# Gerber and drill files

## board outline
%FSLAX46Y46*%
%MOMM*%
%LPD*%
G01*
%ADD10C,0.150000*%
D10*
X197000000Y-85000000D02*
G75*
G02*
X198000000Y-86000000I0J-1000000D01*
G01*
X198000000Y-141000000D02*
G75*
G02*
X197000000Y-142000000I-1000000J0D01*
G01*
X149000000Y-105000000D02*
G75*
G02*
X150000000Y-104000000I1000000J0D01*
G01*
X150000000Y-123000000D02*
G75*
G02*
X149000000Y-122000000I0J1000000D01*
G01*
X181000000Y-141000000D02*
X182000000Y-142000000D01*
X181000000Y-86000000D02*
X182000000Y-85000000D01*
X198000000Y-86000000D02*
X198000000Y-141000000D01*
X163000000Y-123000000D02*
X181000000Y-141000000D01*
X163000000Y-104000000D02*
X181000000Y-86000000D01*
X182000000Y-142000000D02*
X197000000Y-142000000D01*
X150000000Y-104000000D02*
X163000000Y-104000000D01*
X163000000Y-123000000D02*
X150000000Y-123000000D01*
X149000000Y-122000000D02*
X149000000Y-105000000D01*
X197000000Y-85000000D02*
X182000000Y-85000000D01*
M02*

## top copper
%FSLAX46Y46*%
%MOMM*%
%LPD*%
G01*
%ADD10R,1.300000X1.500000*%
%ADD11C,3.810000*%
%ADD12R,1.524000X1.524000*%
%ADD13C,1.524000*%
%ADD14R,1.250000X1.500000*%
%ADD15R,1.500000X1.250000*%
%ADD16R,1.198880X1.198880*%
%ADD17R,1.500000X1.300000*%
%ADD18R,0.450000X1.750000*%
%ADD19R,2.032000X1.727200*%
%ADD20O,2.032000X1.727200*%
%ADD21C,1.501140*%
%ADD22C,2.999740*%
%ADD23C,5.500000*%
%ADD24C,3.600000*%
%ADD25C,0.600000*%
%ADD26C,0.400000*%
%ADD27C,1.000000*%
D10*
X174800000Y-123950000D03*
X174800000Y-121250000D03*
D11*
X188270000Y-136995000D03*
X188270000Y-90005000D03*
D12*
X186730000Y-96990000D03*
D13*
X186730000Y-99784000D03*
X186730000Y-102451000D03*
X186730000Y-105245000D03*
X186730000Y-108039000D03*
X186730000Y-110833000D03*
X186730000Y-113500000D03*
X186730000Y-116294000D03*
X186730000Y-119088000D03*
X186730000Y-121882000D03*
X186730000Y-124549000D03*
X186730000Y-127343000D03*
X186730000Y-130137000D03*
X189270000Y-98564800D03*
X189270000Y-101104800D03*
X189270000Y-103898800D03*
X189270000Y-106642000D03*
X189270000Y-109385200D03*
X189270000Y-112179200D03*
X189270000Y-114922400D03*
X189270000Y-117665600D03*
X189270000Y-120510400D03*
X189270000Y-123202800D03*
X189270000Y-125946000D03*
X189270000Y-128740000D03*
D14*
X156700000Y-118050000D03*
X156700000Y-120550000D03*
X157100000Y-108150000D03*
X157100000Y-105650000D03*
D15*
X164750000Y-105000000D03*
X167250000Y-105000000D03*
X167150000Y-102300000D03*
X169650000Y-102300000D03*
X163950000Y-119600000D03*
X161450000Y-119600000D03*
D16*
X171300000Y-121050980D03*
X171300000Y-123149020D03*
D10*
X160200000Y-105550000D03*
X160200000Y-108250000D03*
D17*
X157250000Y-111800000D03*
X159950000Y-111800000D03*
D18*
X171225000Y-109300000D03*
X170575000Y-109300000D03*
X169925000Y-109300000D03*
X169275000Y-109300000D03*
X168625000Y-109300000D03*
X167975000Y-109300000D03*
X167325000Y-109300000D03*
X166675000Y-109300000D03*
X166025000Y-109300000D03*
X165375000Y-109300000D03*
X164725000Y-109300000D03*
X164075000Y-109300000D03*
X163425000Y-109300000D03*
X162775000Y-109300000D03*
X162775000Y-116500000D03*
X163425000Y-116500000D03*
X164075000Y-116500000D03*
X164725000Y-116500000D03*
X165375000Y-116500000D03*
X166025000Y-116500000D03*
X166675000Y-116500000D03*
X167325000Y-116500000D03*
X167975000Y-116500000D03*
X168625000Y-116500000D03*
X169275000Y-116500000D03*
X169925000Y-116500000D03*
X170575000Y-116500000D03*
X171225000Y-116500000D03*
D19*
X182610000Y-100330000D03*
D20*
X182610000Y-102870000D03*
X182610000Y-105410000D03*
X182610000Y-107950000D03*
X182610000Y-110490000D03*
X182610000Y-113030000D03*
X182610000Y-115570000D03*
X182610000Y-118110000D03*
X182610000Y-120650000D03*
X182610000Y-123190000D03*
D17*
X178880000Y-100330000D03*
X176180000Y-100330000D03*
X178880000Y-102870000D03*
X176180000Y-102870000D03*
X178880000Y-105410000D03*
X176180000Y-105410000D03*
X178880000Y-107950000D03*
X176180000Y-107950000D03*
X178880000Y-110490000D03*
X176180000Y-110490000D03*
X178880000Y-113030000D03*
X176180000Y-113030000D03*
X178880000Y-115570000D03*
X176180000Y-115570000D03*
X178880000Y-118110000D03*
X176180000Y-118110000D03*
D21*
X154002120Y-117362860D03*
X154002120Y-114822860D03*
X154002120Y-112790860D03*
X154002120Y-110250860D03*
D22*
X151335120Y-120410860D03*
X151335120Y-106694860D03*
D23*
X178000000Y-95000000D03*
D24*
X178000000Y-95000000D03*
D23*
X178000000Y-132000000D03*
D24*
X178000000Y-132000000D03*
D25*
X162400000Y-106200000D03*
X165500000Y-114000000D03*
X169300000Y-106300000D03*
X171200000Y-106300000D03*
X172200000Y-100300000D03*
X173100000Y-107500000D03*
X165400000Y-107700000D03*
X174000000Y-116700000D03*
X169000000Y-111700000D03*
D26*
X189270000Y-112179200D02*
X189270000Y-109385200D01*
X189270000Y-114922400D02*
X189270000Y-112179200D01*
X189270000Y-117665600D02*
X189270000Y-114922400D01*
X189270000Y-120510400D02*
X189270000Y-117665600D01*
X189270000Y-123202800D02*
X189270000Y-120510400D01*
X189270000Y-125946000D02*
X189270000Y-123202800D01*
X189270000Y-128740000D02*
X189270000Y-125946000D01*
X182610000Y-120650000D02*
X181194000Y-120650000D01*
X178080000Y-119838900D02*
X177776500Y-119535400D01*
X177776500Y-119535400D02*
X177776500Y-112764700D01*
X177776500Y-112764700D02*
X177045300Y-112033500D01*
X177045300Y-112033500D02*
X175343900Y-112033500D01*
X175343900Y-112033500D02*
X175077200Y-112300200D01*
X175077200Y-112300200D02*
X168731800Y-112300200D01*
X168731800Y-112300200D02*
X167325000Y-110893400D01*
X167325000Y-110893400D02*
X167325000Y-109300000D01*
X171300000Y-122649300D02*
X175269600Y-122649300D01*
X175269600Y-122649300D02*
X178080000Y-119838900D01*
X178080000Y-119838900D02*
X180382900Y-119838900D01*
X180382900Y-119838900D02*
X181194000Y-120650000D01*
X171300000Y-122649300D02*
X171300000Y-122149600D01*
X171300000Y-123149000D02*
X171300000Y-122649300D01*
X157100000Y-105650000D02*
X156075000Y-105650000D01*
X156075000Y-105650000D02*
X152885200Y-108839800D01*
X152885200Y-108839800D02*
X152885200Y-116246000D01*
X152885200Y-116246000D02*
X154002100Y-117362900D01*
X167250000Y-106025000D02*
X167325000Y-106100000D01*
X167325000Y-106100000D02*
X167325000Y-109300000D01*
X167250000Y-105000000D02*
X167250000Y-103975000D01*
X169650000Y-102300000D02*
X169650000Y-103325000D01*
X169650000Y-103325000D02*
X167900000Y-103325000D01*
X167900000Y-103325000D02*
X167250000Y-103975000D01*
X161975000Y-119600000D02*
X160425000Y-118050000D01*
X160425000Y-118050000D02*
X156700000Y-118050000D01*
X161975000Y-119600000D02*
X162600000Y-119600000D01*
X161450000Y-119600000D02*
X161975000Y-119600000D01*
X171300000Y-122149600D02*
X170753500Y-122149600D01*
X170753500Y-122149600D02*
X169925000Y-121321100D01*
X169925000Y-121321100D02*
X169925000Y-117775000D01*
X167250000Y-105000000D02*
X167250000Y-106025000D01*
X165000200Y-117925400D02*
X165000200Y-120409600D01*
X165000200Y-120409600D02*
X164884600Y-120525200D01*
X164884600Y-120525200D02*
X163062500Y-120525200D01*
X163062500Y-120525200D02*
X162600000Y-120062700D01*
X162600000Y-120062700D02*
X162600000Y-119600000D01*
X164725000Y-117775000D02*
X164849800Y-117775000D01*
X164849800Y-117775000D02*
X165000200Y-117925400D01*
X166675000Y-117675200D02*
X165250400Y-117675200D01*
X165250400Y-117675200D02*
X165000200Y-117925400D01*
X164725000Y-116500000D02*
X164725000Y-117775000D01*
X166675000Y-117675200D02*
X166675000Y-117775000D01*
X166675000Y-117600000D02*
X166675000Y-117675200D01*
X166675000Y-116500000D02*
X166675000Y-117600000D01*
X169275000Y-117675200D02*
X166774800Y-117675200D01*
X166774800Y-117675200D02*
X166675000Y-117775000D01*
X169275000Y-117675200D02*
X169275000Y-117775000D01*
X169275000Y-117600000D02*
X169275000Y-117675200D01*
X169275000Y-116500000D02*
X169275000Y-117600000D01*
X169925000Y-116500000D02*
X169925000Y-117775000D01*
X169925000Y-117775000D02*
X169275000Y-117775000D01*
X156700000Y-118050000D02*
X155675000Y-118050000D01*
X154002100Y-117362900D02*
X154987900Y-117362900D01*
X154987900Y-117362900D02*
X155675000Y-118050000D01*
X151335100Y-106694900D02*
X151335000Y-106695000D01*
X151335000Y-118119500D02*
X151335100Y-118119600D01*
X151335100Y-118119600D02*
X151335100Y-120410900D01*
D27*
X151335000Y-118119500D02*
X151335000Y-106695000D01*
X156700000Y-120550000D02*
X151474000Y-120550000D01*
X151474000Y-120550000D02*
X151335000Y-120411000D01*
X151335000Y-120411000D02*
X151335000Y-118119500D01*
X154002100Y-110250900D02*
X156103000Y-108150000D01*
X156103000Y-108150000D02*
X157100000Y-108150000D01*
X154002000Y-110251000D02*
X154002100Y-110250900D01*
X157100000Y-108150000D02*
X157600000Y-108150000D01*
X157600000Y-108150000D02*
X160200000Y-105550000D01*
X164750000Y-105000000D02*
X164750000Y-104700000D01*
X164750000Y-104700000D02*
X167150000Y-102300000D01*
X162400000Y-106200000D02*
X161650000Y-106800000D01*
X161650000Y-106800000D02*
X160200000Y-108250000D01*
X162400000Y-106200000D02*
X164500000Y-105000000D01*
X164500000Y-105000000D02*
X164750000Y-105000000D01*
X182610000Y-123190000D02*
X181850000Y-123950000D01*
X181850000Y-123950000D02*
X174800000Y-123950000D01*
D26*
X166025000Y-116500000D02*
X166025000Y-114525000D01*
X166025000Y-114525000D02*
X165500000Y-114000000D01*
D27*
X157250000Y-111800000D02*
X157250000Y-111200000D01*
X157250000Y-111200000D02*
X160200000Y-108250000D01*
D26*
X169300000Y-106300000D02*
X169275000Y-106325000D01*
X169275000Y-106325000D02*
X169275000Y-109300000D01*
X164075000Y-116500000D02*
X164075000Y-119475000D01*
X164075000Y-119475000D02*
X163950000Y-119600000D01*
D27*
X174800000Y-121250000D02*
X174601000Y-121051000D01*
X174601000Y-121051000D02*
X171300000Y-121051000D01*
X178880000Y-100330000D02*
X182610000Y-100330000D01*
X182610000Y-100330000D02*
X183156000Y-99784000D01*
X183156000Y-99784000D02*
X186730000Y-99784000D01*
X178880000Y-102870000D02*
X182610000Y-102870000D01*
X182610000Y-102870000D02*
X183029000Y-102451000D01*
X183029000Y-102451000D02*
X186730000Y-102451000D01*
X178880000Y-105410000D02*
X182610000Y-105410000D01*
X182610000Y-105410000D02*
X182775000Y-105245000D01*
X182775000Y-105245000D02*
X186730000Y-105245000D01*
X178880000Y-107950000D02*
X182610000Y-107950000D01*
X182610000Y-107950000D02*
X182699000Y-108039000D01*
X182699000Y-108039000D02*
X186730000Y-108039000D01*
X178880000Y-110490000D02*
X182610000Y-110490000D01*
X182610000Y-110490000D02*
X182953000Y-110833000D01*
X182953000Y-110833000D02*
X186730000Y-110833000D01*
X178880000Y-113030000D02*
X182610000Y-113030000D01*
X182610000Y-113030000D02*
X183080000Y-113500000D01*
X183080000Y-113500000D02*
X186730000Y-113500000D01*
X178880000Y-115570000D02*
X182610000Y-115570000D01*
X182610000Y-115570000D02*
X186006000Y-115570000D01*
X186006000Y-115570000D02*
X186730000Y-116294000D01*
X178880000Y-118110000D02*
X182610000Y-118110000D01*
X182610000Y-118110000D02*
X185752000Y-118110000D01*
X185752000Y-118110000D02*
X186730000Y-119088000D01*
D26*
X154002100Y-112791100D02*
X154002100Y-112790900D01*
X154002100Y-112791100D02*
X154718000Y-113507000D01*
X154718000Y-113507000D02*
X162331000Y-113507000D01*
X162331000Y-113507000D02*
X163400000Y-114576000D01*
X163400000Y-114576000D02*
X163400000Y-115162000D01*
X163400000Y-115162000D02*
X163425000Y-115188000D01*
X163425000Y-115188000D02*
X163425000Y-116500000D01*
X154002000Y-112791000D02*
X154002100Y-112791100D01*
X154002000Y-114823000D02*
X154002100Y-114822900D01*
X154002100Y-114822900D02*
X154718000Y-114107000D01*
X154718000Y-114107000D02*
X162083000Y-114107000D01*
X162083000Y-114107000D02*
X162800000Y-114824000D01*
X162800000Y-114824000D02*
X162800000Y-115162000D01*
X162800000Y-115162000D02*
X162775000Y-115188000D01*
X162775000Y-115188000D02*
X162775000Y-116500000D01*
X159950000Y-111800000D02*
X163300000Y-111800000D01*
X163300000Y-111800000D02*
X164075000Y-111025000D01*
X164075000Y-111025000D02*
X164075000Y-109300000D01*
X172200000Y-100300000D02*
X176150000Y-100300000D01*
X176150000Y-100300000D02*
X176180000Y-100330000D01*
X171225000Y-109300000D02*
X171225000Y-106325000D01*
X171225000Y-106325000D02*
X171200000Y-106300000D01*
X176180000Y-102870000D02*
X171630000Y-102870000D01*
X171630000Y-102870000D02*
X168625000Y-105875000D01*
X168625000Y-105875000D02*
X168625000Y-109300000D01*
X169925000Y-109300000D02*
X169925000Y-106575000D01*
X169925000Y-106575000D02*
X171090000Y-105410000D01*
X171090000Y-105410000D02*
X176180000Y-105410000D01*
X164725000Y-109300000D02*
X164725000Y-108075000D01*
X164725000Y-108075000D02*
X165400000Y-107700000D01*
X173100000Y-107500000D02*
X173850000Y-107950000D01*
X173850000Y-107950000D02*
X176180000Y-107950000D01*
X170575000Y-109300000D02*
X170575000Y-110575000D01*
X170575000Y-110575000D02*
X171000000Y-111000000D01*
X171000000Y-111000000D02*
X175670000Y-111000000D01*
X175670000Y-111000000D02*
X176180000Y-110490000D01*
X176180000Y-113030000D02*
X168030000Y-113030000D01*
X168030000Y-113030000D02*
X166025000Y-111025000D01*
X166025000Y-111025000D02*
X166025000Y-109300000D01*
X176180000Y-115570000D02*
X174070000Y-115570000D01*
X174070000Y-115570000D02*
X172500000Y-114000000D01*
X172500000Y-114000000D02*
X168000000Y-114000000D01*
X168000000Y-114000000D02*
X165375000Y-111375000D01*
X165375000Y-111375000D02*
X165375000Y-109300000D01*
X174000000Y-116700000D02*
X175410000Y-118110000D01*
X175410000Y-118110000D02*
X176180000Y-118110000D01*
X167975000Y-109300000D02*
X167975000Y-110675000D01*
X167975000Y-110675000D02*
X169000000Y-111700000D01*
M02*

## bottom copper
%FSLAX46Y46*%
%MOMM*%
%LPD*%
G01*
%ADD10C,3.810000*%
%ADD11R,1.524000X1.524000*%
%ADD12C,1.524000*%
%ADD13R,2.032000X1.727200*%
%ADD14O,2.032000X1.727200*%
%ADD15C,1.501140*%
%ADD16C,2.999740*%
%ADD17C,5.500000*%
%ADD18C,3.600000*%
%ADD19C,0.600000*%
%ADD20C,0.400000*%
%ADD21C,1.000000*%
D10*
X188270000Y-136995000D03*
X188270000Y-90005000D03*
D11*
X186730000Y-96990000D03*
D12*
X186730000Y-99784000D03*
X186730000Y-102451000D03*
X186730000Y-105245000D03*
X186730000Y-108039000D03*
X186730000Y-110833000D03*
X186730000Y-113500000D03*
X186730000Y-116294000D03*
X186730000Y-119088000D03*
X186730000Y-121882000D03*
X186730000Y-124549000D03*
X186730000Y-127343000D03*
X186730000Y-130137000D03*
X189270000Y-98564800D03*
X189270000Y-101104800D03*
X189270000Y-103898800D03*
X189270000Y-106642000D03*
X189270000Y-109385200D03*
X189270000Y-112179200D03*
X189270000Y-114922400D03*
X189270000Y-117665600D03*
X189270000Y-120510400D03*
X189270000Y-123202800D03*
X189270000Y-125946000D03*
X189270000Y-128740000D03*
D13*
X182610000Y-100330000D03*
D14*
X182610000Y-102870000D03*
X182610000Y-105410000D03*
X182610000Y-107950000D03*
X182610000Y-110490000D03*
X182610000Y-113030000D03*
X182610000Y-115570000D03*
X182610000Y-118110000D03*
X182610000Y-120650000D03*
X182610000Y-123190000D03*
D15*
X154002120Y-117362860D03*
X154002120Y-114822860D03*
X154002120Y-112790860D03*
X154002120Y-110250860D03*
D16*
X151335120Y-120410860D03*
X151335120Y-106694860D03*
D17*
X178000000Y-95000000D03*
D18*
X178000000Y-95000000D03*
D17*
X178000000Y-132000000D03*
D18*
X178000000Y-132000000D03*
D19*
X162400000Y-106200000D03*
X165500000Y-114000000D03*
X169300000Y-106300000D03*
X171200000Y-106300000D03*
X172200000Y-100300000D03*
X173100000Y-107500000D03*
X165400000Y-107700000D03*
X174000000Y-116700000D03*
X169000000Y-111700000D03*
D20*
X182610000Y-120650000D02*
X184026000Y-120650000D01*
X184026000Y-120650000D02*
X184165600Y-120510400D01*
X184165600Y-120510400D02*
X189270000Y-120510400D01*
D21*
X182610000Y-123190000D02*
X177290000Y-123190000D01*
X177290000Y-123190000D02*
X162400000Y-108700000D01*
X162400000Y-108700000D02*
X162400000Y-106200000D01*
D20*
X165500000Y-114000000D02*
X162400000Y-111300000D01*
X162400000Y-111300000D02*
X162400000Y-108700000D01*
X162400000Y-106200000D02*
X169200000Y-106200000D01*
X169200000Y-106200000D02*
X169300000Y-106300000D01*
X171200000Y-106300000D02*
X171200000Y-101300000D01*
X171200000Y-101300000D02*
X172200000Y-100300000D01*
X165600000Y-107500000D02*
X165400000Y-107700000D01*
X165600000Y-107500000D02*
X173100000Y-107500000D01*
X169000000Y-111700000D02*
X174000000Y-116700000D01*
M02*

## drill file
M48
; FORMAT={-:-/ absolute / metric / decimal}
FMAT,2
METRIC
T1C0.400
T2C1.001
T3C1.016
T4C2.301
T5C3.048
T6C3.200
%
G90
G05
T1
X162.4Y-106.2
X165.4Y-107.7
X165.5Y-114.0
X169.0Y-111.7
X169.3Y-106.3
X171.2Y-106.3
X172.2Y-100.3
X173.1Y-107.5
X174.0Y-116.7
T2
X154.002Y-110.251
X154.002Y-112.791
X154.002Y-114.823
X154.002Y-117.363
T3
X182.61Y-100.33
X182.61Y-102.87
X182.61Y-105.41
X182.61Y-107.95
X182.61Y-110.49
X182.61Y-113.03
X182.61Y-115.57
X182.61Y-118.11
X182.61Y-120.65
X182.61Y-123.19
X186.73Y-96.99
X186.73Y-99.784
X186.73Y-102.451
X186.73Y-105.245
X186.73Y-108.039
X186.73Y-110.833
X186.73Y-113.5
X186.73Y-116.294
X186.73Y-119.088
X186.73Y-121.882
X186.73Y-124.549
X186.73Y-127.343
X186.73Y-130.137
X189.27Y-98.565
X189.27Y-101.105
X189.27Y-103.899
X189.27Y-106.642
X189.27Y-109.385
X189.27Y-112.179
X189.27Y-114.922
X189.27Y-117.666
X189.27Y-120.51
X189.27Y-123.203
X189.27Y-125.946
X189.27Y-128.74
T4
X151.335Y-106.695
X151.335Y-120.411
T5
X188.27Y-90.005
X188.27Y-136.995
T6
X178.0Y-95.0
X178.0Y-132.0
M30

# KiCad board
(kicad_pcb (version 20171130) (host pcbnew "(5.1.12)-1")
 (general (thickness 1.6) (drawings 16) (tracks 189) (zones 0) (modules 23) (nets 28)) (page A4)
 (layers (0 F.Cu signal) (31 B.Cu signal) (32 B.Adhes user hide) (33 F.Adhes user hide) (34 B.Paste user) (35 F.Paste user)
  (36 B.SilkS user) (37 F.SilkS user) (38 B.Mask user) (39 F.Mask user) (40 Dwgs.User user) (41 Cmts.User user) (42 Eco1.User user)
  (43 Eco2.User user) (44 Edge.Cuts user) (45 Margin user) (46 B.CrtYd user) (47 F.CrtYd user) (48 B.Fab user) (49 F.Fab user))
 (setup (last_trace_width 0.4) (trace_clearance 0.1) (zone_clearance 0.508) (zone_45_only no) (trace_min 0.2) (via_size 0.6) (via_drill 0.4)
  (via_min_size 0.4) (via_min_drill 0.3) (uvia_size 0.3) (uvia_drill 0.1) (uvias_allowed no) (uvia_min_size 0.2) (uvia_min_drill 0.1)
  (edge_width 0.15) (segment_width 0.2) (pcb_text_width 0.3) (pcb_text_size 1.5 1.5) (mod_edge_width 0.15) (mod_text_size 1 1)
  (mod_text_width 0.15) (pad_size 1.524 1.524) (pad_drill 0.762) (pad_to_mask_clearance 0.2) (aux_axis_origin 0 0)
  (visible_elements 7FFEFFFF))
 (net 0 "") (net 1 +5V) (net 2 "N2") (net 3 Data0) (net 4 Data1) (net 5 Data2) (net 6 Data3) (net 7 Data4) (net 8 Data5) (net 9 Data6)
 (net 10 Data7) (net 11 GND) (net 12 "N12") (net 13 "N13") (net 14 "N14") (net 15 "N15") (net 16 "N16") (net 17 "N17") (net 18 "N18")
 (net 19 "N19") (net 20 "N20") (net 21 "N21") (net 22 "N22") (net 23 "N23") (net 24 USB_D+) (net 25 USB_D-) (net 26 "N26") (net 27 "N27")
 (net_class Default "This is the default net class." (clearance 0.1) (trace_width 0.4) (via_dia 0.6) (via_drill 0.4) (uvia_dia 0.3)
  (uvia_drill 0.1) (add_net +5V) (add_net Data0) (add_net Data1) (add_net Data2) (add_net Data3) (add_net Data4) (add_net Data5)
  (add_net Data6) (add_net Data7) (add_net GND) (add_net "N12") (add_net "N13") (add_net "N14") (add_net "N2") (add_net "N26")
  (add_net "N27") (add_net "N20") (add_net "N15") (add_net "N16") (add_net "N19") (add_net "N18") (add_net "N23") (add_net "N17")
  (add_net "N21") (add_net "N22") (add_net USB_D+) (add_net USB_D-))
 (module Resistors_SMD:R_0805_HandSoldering (layer F.Cu) (at 174.8 122.6 90)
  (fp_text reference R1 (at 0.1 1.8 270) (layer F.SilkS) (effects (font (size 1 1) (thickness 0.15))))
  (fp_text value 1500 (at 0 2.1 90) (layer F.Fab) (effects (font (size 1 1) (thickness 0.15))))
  (pad 1 smd rect (at -1.35 0 90) (size 1.5 1.3) (layers F.Cu F.Paste F.Mask) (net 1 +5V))
  (pad 2 smd rect (at 1.35 0 90) (size 1.5 1.3) (layers F.Cu F.Paste F.Mask) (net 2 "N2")))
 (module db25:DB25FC (layer F.Cu) (at 187 113.5 270)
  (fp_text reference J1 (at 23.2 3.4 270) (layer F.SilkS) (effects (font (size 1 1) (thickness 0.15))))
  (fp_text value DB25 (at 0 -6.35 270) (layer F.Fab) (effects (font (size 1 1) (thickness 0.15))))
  (pad "" thru_hole circle (at 23.495 -1.27 270) (size 3.81 3.81) (drill 3.048) (layers *.Cu *.Mask F.SilkS))
  (pad "" thru_hole circle (at -23.495 -1.27 270) (size 3.81 3.81) (drill 3.048) (layers *.Cu *.Mask F.SilkS))
  (pad 1 thru_hole rect (at -16.51 0.27 270) (size 1.524 1.524) (drill 1.016) (layers *.Cu *.Mask F.SilkS))
  (pad 2 thru_hole circle (at -13.716 0.27 270) (size 1.524 1.524) (drill 1.016) (layers *.Cu *.Mask F.SilkS) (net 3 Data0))
  (pad 3 thru_hole circle (at -11.049 0.27 270) (size 1.524 1.524) (drill 1.016) (layers *.Cu *.Mask F.SilkS) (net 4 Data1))
  (pad 4 thru_hole circle (at -8.255 0.27 270) (size 1.524 1.524) (drill 1.016) (layers *.Cu *.Mask F.SilkS) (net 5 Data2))
  (pad 5 thru_hole circle (at -5.461 0.27 270) (size 1.524 1.524) (drill 1.016) (layers *.Cu *.Mask F.SilkS) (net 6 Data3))
  (pad 6 thru_hole circle (at -2.667 0.27 270) (size 1.524 1.524) (drill 1.016) (layers *.Cu *.Mask F.SilkS) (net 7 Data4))
  (pad 7 thru_hole circle (at 0 0.27 270) (size 1.524 1.524) (drill 1.016) (layers *.Cu *.Mask F.SilkS) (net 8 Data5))
  (pad 8 thru_hole circle (at 2.794 0.27 270) (size 1.524 1.524) (drill 1.016) (layers *.Cu *.Mask F.SilkS) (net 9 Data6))
  (pad 9 thru_hole circle (at 5.588 0.27 270) (size 1.524 1.524) (drill 1.016) (layers *.Cu *.Mask F.SilkS) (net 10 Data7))
  (pad 10 thru_hole circle (at 8.382 0.27 270) (size 1.524 1.524) (drill 1.016) (layers *.Cu *.Mask F.SilkS))
  (pad 11 thru_hole circle (at 11.049 0.27 270) (size 1.524 1.524) (drill 1.016) (layers *.Cu *.Mask F.SilkS))
  (pad 12 thru_hole circle (at 13.843 0.27 270) (size 1.524 1.524) (drill 1.016) (layers *.Cu *.Mask F.SilkS))
  (pad 13 thru_hole circle (at 16.637 0.27 270) (size 1.524 1.524) (drill 1.016) (layers *.Cu *.Mask F.SilkS))
  (pad 14 thru_hole circle (at -14.9352 -2.27 270) (size 1.524 1.524) (drill 1.016) (layers *.Cu *.Mask F.SilkS))
  (pad 15 thru_hole circle (at -12.3952 -2.27 270) (size 1.524 1.524) (drill 1.016) (layers *.Cu *.Mask F.SilkS))
  (pad 16 thru_hole circle (at -9.6012 -2.27 270) (size 1.524 1.524) (drill 1.016) (layers *.Cu *.Mask F.SilkS))
  (pad 17 thru_hole circle (at -6.858 -2.27 270) (size 1.524 1.524) (drill 1.016) (layers *.Cu *.Mask F.SilkS))
  (pad 18 thru_hole circle (at -4.1148 -2.27 270) (size 1.524 1.524) (drill 1.016) (layers *.Cu *.Mask F.SilkS) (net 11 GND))
  (pad 19 thru_hole circle (at -1.3208 -2.27 270) (size 1.524 1.524) (drill 1.016) (layers *.Cu *.Mask F.SilkS) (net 11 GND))
  (pad 20 thru_hole circle (at 1.4224 -2.27 270) (size 1.524 1.524) (drill 1.016) (layers *.Cu *.Mask F.SilkS) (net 11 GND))
  (pad 21 thru_hole circle (at 4.1656 -2.27 270) (size 1.524 1.524) (drill 1.016) (layers *.Cu *.Mask F.SilkS) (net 11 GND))
  (pad 22 thru_hole circle (at 7.0104 -2.27 270) (size 1.524 1.524) (drill 1.016) (layers *.Cu *.Mask F.SilkS) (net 11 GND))
  (pad 23 thru_hole circle (at 9.7028 -2.27 270) (size 1.524 1.524) (drill 1.016) (layers *.Cu *.Mask F.SilkS) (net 11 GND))
  (pad 24 thru_hole circle (at 12.446 -2.27 270) (size 1.524 1.524) (drill 1.016) (layers *.Cu *.Mask F.SilkS) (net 11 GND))
  (pad 25 thru_hole circle (at 15.24 -2.27 270) (size 1.524 1.524) (drill 1.016) (layers *.Cu *.Mask F.SilkS) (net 11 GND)))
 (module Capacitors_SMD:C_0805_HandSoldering (layer F.Cu) (at 156.7 119.3 270)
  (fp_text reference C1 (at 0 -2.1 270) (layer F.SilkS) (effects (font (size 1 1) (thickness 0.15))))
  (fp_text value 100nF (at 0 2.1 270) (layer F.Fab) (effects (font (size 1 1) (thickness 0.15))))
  (pad 1 smd rect (at -1.25 0 270) (size 1.5 1.25) (layers F.Cu F.Paste F.Mask) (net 11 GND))
  (pad 2 smd rect (at 1.25 0 270) (size 1.5 1.25) (layers F.Cu F.Paste F.Mask) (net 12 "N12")))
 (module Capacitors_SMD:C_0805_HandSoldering (layer F.Cu) (at 157.1 106.9 90)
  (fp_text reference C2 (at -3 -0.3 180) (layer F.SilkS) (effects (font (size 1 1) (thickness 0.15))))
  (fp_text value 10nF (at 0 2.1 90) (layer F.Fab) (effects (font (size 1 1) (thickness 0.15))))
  (pad 1 smd rect (at -1.25 0 90) (size 1.5 1.25) (layers F.Cu F.Paste F.Mask) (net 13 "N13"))
  (pad 2 smd rect (at 1.25 0 90) (size 1.5 1.25) (layers F.Cu F.Paste F.Mask) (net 11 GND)))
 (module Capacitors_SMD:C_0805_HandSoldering (layer F.Cu) (at 166 105)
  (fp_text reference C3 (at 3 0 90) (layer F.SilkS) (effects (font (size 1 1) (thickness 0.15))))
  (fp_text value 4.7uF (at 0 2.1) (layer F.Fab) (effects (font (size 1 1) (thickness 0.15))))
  (pad 1 smd rect (at -1.25 0) (size 1.5 1.25) (layers F.Cu F.Paste F.Mask) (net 1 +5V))
  (pad 2 smd rect (at 1.25 0) (size 1.5 1.25) (layers F.Cu F.Paste F.Mask) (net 11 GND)))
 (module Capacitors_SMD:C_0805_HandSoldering (layer F.Cu) (at 168.4 102.3)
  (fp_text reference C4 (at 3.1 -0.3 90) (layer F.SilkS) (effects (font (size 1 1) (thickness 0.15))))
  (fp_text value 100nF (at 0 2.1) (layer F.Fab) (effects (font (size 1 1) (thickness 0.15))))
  (pad 1 smd rect (at -1.25 0) (size 1.5 1.25) (layers F.Cu F.Paste F.Mask) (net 1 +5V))
  (pad 2 smd rect (at 1.25 0) (size 1.5 1.25) (layers F.Cu F.Paste F.Mask) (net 11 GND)))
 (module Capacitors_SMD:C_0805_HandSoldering (layer F.Cu) (at 162.7 119.6 180)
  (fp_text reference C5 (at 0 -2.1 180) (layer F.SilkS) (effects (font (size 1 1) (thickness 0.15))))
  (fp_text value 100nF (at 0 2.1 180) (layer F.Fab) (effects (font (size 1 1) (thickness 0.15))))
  (pad 1 smd rect (at -1.25 0 180) (size 1.5 1.25) (layers F.Cu F.Paste F.Mask) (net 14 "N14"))
  (pad 2 smd rect (at 1.25 0 180) (size 1.5 1.25) (layers F.Cu F.Paste F.Mask) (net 11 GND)))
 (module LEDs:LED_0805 (layer F.Cu) (at 171.3 122.1 90)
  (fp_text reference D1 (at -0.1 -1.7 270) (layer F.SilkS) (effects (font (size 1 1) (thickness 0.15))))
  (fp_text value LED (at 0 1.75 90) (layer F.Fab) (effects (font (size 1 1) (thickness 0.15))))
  (pad 2 smd rect (at 1.04902 0 270) (size 1.19888 1.19888) (layers F.Cu F.Paste F.Mask) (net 2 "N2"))
  (pad 1 smd rect (at -1.04902 0 270) (size 1.19888 1.19888) (layers F.Cu F.Paste F.Mask) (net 11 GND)))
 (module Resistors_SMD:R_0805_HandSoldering (layer F.Cu) (at 160.2 106.9 270)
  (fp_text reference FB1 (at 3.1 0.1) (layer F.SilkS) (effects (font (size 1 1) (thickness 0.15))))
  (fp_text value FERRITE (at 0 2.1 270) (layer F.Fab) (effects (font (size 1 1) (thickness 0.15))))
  (pad 1 smd rect (at -1.35 0 270) (size 1.5 1.3) (layers F.Cu F.Paste F.Mask) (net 13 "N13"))
  (pad 2 smd rect (at 1.35 0 270) (size 1.5 1.3) (layers F.Cu F.Paste F.Mask) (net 1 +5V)))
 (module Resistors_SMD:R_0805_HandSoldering (layer F.Cu) (at 158.6 111.8)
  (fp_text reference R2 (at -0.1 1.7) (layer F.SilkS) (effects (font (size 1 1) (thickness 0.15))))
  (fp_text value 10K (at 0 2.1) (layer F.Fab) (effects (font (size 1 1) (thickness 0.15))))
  (pad 1 smd rect (at -1.35 0) (size 1.5 1.3) (layers F.Cu F.Paste F.Mask) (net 1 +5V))
  (pad 2 smd rect (at 1.35 0) (size 1.5 1.3) (layers F.Cu F.Paste F.Mask) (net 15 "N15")))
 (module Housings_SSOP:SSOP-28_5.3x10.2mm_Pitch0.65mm (layer F.Cu) (at 167 112.9 270)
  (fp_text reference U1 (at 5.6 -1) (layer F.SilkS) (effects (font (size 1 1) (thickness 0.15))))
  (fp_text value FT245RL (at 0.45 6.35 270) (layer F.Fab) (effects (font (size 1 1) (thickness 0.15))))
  (pad 1 smd rect (at -3.6 -4.225 270) (size 1.75 0.45) (layers F.Cu F.Paste F.Mask) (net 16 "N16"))
  (pad 2 smd rect (at -3.6 -3.575 270) (size 1.75 0.45) (layers F.Cu F.Paste F.Mask) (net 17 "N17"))
  (pad 3 smd rect (at -3.6 -2.925 270) (size 1.75 0.45) (layers F.Cu F.Paste F.Mask) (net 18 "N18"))
  (pad 4 smd rect (at -3.6 -2.275 270) (size 1.75 0.45) (layers F.Cu F.Paste F.Mask) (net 1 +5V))
  (pad 5 smd rect (at -3.6 -1.625 270) (size 1.75 0.45) (layers F.Cu F.Paste F.Mask) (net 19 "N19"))
  (pad 6 smd rect (at -3.6 -0.975 270) (size 1.75 0.45) (layers F.Cu F.Paste F.Mask) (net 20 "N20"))
  (pad 7 smd rect (at -3.6 -0.325 270) (size 1.75 0.45) (layers F.Cu F.Paste F.Mask) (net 11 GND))
  (pad 8 smd rect (at -3.6 0.325 270) (size 1.75 0.45) (layers F.Cu F.Paste F.Mask))
  (pad 9 smd rect (at -3.6 0.975 270) (size 1.75 0.45) (layers F.Cu F.Paste F.Mask) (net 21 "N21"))
  (pad 10 smd rect (at -3.6 1.625 270) (size 1.75 0.45) (layers F.Cu F.Paste F.Mask) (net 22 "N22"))
  (pad 11 smd rect (at -3.6 2.275 270) (size 1.75 0.45) (layers F.Cu F.Paste F.Mask) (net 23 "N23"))
  (pad 12 smd rect (at -3.6 2.925 270) (size 1.75 0.45) (layers F.Cu F.Paste F.Mask) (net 15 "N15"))
  (pad 13 smd rect (at -3.6 3.575 270) (size 1.75 0.45) (layers F.Cu F.Paste F.Mask))
  (pad 14 smd rect (at -3.6 4.225 270) (size 1.75 0.45) (layers F.Cu F.Paste F.Mask))
  (pad 15 smd rect (at 3.6 4.225 270) (size 1.75 0.45) (layers F.Cu F.Paste F.Mask) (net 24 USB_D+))
  (pad 16 smd rect (at 3.6 3.575 270) (size 1.75 0.45) (layers F.Cu F.Paste F.Mask) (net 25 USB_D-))
  (pad 17 smd rect (at 3.6 2.925 270) (size 1.75 0.45) (layers F.Cu F.Paste F.Mask) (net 14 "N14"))
  (pad 18 smd rect (at 3.6 2.275 270) (size 1.75 0.45) (layers F.Cu F.Paste F.Mask) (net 11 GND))
  (pad 19 smd rect (at 3.6 1.625 270) (size 1.75 0.45) (layers F.Cu F.Paste F.Mask))
  (pad 20 smd rect (at 3.6 0.975 270) (size 1.75 0.45) (layers F.Cu F.Paste F.Mask) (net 1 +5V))
  (pad 21 smd rect (at 3.6 0.325 270) (size 1.75 0.45) (layers F.Cu F.Paste F.Mask) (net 11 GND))
  (pad 22 smd rect (at 3.6 -0.325 270) (size 1.75 0.45) (layers F.Cu F.Paste F.Mask))
  (pad 23 smd rect (at 3.6 -0.975 270) (size 1.75 0.45) (layers F.Cu F.Paste F.Mask))
  (pad 24 smd rect (at 3.6 -1.625 270) (size 1.75 0.45) (layers F.Cu F.Paste F.Mask))
  (pad 25 smd rect (at 3.6 -2.275 270) (size 1.75 0.45) (layers F.Cu F.Paste F.Mask) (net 11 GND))
  (pad 26 smd rect (at 3.6 -2.925 270) (size 1.75 0.45) (layers F.Cu F.Paste F.Mask) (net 11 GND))
  (pad 27 smd rect (at 3.6 -3.575 270) (size 1.75 0.45) (layers F.Cu F.Paste F.Mask))
  (pad 28 smd rect (at 3.6 -4.225 270) (size 1.75 0.45) (layers F.Cu F.Paste F.Mask)))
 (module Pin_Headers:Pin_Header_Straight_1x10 (layer F.Cu) (at 182.61 100.33)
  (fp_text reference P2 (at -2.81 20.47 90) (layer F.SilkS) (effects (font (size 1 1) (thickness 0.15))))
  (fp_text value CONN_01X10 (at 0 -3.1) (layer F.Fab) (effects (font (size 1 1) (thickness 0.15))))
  (pad 1 thru_hole rect (at 0 0) (size 2.032 1.7272) (drill 1.016) (layers *.Cu *.Mask F.SilkS) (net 3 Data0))
  (pad 2 thru_hole oval (at 0 2.54) (size 2.032 1.7272) (drill 1.016) (layers *.Cu *.Mask F.SilkS) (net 4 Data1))
  (pad 3 thru_hole oval (at 0 5.08) (size 2.032 1.7272) (drill 1.016) (layers *.Cu *.Mask F.SilkS) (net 5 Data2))
  (pad 4 thru_hole oval (at 0 7.62) (size 2.032 1.7272) (drill 1.016) (layers *.Cu *.Mask F.SilkS) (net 6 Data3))
  (pad 5 thru_hole oval (at 0 10.16) (size 2.032 1.7272) (drill 1.016) (layers *.Cu *.Mask F.SilkS) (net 7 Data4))
  (pad 6 thru_hole oval (at 0 12.7) (size 2.032 1.7272) (drill 1.016) (layers *.Cu *.Mask F.SilkS) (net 8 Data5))
  (pad 7 thru_hole oval (at 0 15.24) (size 2.032 1.7272) (drill 1.016) (layers *.Cu *.Mask F.SilkS) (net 9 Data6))
  (pad 8 thru_hole oval (at 0 17.78) (size 2.032 1.7272) (drill 1.016) (layers *.Cu *.Mask F.SilkS) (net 10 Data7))
  (pad 9 thru_hole oval (at 0 20.32) (size 2.032 1.7272) (drill 1.016) (layers *.Cu *.Mask F.SilkS) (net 11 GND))
  (pad 10 thru_hole oval (at 0 22.86) (size 2.032 1.7272) (drill 1.016) (layers *.Cu *.Mask F.SilkS) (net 1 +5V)))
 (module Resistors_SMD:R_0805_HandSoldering (layer F.Cu) (at 177.53 100.33 180)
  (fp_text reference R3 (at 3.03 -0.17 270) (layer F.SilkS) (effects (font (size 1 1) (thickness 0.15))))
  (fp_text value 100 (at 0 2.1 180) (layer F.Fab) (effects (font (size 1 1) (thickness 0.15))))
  (pad 1 smd rect (at -1.35 0 180) (size 1.5 1.3) (layers F.Cu F.Paste F.Mask) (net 3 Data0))
  (pad 2 smd rect (at 1.35 0 180) (size 1.5 1.3) (layers F.Cu F.Paste F.Mask) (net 16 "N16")))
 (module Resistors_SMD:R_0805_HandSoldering (layer F.Cu) (at 177.53 102.87 180)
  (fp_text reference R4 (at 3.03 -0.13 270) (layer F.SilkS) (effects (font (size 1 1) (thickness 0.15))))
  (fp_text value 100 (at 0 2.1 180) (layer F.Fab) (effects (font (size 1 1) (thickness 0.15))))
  (pad 1 smd rect (at -1.35 0 180) (size 1.5 1.3) (layers F.Cu F.Paste F.Mask) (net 4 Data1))
  (pad 2 smd rect (at 1.35 0 180) (size 1.5 1.3) (layers F.Cu F.Paste F.Mask) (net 19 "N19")))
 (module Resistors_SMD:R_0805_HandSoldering (layer F.Cu) (at 177.53 105.41 180)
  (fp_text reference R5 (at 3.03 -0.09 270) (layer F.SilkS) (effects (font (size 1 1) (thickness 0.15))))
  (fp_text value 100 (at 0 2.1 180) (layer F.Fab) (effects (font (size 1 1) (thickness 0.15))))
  (pad 1 smd rect (at -1.35 0 180) (size 1.5 1.3) (layers F.Cu F.Paste F.Mask) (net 5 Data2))
  (pad 2 smd rect (at 1.35 0 180) (size 1.5 1.3) (layers F.Cu F.Paste F.Mask) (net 18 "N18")))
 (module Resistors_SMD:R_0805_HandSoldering (layer F.Cu) (at 177.53 107.95 180)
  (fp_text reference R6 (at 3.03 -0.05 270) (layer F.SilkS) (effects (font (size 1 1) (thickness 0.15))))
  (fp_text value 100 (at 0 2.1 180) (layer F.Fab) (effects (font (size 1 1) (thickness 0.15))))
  (pad 1 smd rect (at -1.35 0 180) (size 1.5 1.3) (layers F.Cu F.Paste F.Mask) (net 6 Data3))
  (pad 2 smd rect (at 1.35 0 180) (size 1.5 1.3) (layers F.Cu F.Paste F.Mask) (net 23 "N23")))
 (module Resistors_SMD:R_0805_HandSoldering (layer F.Cu) (at 177.53 110.49 180)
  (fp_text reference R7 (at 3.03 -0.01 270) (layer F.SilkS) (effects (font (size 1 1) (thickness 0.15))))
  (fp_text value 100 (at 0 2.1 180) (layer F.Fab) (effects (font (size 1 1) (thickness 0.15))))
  (pad 1 smd rect (at -1.35 0 180) (size 1.5 1.3) (layers F.Cu F.Paste F.Mask) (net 7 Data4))
  (pad 2 smd rect (at 1.35 0 180) (size 1.5 1.3) (layers F.Cu F.Paste F.Mask) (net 17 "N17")))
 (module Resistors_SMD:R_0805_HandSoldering (layer F.Cu) (at 177.53 113.03 180)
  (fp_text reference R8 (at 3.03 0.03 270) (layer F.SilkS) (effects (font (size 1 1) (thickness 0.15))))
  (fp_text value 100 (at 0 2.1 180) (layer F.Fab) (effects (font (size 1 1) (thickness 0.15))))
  (pad 1 smd rect (at -1.35 0 180) (size 1.5 1.3) (layers F.Cu F.Paste F.Mask) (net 8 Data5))
  (pad 2 smd rect (at 1.35 0 180) (size 1.5 1.3) (layers F.Cu F.Paste F.Mask) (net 21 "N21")))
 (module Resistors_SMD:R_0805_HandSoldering (layer F.Cu) (at 177.53 115.57 180)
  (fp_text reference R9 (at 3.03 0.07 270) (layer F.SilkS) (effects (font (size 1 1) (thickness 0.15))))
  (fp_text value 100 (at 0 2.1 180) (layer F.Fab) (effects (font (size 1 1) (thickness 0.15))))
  (pad 1 smd rect (at -1.35 0 180) (size 1.5 1.3) (layers F.Cu F.Paste F.Mask) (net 9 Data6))
  (pad 2 smd rect (at 1.35 0 180) (size 1.5 1.3) (layers F.Cu F.Paste F.Mask) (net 22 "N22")))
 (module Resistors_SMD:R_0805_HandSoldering (layer F.Cu) (at 177.53 118.11 180)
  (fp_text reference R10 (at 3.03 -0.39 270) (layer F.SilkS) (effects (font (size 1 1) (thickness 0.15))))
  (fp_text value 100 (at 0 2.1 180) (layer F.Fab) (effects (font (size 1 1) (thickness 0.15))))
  (pad 1 smd rect (at -1.35 0 180) (size 1.5 1.3) (layers F.Cu F.Paste F.Mask) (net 10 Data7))
  (pad 2 smd rect (at 1.35 0 180) (size 1.5 1.3) (layers F.Cu F.Paste F.Mask) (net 20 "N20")))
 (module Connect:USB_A (layer F.Cu) (at 154 110.25 270)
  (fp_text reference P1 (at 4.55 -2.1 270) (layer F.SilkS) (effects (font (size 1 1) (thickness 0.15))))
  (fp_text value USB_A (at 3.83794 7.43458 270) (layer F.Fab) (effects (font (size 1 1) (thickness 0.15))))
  (pad 4 thru_hole circle (at 7.11286 -0.00212 180) (size 1.50114 1.50114) (drill 1.00076) (layers *.Cu *.Mask F.SilkS) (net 11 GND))
  (pad 3 thru_hole circle (at 4.57286 -0.00212 180) (size 1.50114 1.50114) (drill 1.00076) (layers *.Cu *.Mask F.SilkS) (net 24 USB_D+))
  (pad 2 thru_hole circle (at 2.54086 -0.00212 180) (size 1.50114 1.50114) (drill 1.00076) (layers *.Cu *.Mask F.SilkS) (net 25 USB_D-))
  (pad 1 thru_hole circle (at 0.00086 -0.00212 180) (size 1.50114 1.50114) (drill 1.00076) (layers *.Cu *.Mask F.SilkS) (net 13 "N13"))
  (pad 5 thru_hole circle (at 10.16086 2.66488 180) (size 2.99974 2.99974) (drill 2.30124) (layers *.Cu *.Mask F.SilkS) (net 12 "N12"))
  (pad 5 thru_hole circle (at -3.55514 2.66488 180) (size 2.99974 2.99974) (drill 2.30124) (layers *.Cu *.Mask F.SilkS) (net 12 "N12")))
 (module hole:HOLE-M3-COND (layer F.Cu) (at 178 95)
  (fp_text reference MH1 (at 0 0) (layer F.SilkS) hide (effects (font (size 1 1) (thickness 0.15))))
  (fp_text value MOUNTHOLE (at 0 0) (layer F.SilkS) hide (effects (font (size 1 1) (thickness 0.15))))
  (pad 1 smd circle (at 0 0) (size 5.5 5.5) (layers F.Cu F.Mask) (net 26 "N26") (clearance 0.3) (zone_connect 2))
  (pad 1 smd circle (at 0 0) (size 5.5 5.5) (layers B.Cu B.Mask) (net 26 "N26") (clearance 0.3) (zone_connect 2))
  (pad 1 thru_hole circle (at 0 0) (size 3.6 3.6) (drill 3.2) (layers *.Cu) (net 26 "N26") (clearance 0.2) (zone_connect 2)))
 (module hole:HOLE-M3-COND (layer F.Cu) (at 178 132)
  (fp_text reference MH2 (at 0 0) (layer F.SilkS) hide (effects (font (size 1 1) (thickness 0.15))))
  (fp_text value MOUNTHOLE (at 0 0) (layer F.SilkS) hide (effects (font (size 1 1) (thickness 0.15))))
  (pad 1 smd circle (at 0 0) (size 5.5 5.5) (layers F.Cu F.Mask) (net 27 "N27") (clearance 0.3) (zone_connect 2))
  (pad 1 smd circle (at 0 0) (size 5.5 5.5) (layers B.Cu B.Mask) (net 27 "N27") (clearance 0.3) (zone_connect 2))
  (pad 1 thru_hole circle (at 0 0) (size 3.6 3.6) (drill 3.2) (layers *.Cu) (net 27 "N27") (clearance 0.2) (zone_connect 2)))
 (gr_arc (start 197 86) (end 197 85) (angle 90) (layer Edge.Cuts) (width 0.15))
 (gr_arc (start 197 141) (end 198 141) (angle 90) (layer Edge.Cuts) (width 0.15))
 (gr_arc (start 150 105) (end 149 105) (angle 90) (layer Edge.Cuts) (width 0.15))
 (gr_arc (start 150 122) (end 150 123) (angle 90) (layer Edge.Cuts) (width 0.15))
 (gr_line (start 181 141) (end 182 142) (angle 90) (layer Edge.Cuts) (width 0.15))
 (gr_line (start 181 86) (end 182 85) (angle 90) (layer Edge.Cuts) (width 0.15))
 (gr_line (start 198 86) (end 198 141) (angle 90) (layer Edge.Cuts) (width 0.15))
 (gr_line (start 163 123) (end 181 141) (angle 90) (layer Edge.Cuts) (width 0.15))
 (gr_line (start 163 104) (end 181 86) (angle 90) (layer Edge.Cuts) (width 0.15))
 (gr_line (start 182 142) (end 197 142) (angle 90) (layer Edge.Cuts) (width 0.15))
 (gr_line (start 150 104) (end 163 104) (angle 90) (layer Edge.Cuts) (width 0.15))
 (gr_line (start 163 123) (end 150 123) (angle 90) (layer Edge.Cuts) (width 0.15))
 (gr_line (start 149 122) (end 149 105) (angle 90) (layer Edge.Cuts) (width 0.15))
 (gr_line (start 197 85) (end 182 85) (angle 90) (layer Edge.Cuts) (width 0.15))
 (segment (start 189.27 112.1792) (end 189.27 109.3852) (width 0.4) (layer F.Cu) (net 11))
 (segment (start 189.27 114.9224) (end 189.27 112.1792) (width 0.4) (layer F.Cu) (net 11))
 (segment (start 189.27 117.6656) (end 189.27 114.9224) (width 0.4) (layer F.Cu) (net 11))
 (segment (start 189.27 120.5104) (end 189.27 117.6656) (width 0.4) (layer F.Cu) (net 11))
 (segment (start 189.27 123.2028) (end 189.27 120.5104) (width 0.4) (layer F.Cu) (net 11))
 (segment (start 189.27 125.946) (end 189.27 123.2028) (width 0.4) (layer F.Cu) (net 11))
 (segment (start 189.27 128.74) (end 189.27 125.946) (width 0.4) (layer F.Cu) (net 11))
 (segment (start 182.61 120.65) (end 181.194 120.65) (width 0.4) (layer F.Cu) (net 11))
 (segment (start 178.08 119.8389) (end 177.7765 119.5354) (width 0.4) (layer F.Cu) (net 11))
 (segment (start 177.7765 119.5354) (end 177.7765 112.7647) (width 0.4) (layer F.Cu) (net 11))
 (segment (start 177.7765 112.7647) (end 177.0453 112.0335) (width 0.4) (layer F.Cu) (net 11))
 (segment (start 177.0453 112.0335) (end 175.3439 112.0335) (width 0.4) (layer F.Cu) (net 11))
 (segment (start 175.3439 112.0335) (end 175.0772 112.3002) (width 0.4) (layer F.Cu) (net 11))
 (segment (start 175.0772 112.3002) (end 168.7318 112.3002) (width 0.4) (layer F.Cu) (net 11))
 (segment (start 168.7318 112.3002) (end 167.325 110.8934) (width 0.4) (layer F.Cu) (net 11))
 (segment (start 167.325 110.8934) (end 167.325 109.3) (width 0.4) (layer F.Cu) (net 11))
 (segment (start 171.3 122.6493) (end 175.2696 122.6493) (width 0.4) (layer F.Cu) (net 11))
 (segment (start 175.2696 122.6493) (end 178.08 119.8389) (width 0.4) (layer F.Cu) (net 11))
 (segment (start 178.08 119.8389) (end 180.3829 119.8389) (width 0.4) (layer F.Cu) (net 11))
 (segment (start 180.3829 119.8389) (end 181.194 120.65) (width 0.4) (layer F.Cu) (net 11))
 (segment (start 171.3 122.6493) (end 171.3 122.1496) (width 0.4) (layer F.Cu) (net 11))
 (segment (start 171.3 123.149) (end 171.3 122.6493) (width 0.4) (layer F.Cu) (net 11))
 (segment (start 157.1 105.65) (end 156.075 105.65) (width 0.4) (layer F.Cu) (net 11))
 (segment (start 156.075 105.65) (end 152.8852 108.8398) (width 0.4) (layer F.Cu) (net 11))
 (segment (start 152.8852 108.8398) (end 152.8852 116.246) (width 0.4) (layer F.Cu) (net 11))
 (segment (start 152.8852 116.246) (end 154.0021 117.3629) (width 0.4) (layer F.Cu) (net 11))
 (segment (start 167.25 106.025) (end 167.325 106.1) (width 0.4) (layer F.Cu) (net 11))
 (segment (start 167.325 106.1) (end 167.325 109.3) (width 0.4) (layer F.Cu) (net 11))
 (segment (start 167.25 105) (end 167.25 103.975) (width 0.4) (layer F.Cu) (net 11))
 (segment (start 169.65 102.3) (end 169.65 103.325) (width 0.4) (layer F.Cu) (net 11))
 (segment (start 169.65 103.325) (end 167.9 103.325) (width 0.4) (layer F.Cu) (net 11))
 (segment (start 167.9 103.325) (end 167.25 103.975) (width 0.4) (layer F.Cu) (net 11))
 (segment (start 161.975 119.6) (end 160.425 118.05) (width 0.4) (layer F.Cu) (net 11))
 (segment (start 160.425 118.05) (end 156.7 118.05) (width 0.4) (layer F.Cu) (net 11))
 (segment (start 161.975 119.6) (end 162.6 119.6) (width 0.4) (layer F.Cu) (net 11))
 (segment (start 161.45 119.6) (end 161.975 119.6) (width 0.4) (layer F.Cu) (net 11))
 (segment (start 171.3 122.1496) (end 170.7535 122.1496) (width 0.4) (layer F.Cu) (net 11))
 (segment (start 170.7535 122.1496) (end 169.925 121.3211) (width 0.4) (layer F.Cu) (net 11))
 (segment (start 169.925 121.3211) (end 169.925 117.775) (width 0.4) (layer F.Cu) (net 11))
 (segment (start 167.25 105) (end 167.25 106.025) (width 0.4) (layer F.Cu) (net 11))
 (segment (start 165.0002 117.9254) (end 165.0002 120.4096) (width 0.4) (layer F.Cu) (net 11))
 (segment (start 165.0002 120.4096) (end 164.8846 120.5252) (width 0.4) (layer F.Cu) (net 11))
 (segment (start 164.8846 120.5252) (end 163.0625 120.5252) (width 0.4) (layer F.Cu) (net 11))
 (segment (start 163.0625 120.5252) (end 162.6 120.0627) (width 0.4) (layer F.Cu) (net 11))
 (segment (start 162.6 120.0627) (end 162.6 119.6) (width 0.4) (layer F.Cu) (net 11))
 (segment (start 164.725 117.775) (end 164.8498 117.775) (width 0.4) (layer F.Cu) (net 11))
 (segment (start 164.8498 117.775) (end 165.0002 117.9254) (width 0.4) (layer F.Cu) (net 11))
 (segment (start 166.675 117.6752) (end 165.2504 117.6752) (width 0.4) (layer F.Cu) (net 11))
 (segment (start 165.2504 117.6752) (end 165.0002 117.9254) (width 0.4) (layer F.Cu) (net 11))
 (segment (start 164.725 116.5) (end 164.725 117.775) (width 0.4) (layer F.Cu) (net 11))
 (segment (start 166.675 117.6752) (end 166.675 117.775) (width 0.4) (layer F.Cu) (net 11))
 (segment (start 166.675 117.6) (end 166.675 117.6752) (width 0.4) (layer F.Cu) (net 11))
 (segment (start 166.675 116.5) (end 166.675 117.6) (width 0.4) (layer F.Cu) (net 11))
 (segment (start 169.275 117.6752) (end 166.7748 117.6752) (width 0.4) (layer F.Cu) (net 11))
 (segment (start 166.7748 117.6752) (end 166.675 117.775) (width 0.4) (layer F.Cu) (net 11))
 (segment (start 169.275 117.6752) (end 169.275 117.775) (width 0.4) (layer F.Cu) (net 11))
 (segment (start 169.275 117.6) (end 169.275 117.6752) (width 0.4) (layer F.Cu) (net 11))
 (segment (start 169.275 116.5) (end 169.275 117.6) (width 0.4) (layer F.Cu) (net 11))
 (segment (start 169.925 116.5) (end 169.925 117.775) (width 0.4) (layer F.Cu) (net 11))
 (segment (start 169.925 117.775) (end 169.275 117.775) (width 0.4) (layer F.Cu) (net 11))
 (segment (start 182.61 120.65) (end 184.026 120.65) (width 0.4) (layer B.Cu) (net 11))
 (segment (start 184.026 120.65) (end 184.1656 120.5104) (width 0.4) (layer B.Cu) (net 11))
 (segment (start 184.1656 120.5104) (end 189.27 120.5104) (width 0.4) (layer B.Cu) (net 11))
 (segment (start 156.7 118.05) (end 155.675 118.05) (width 0.4) (layer F.Cu) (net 11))
 (segment (start 154.0021 117.3629) (end 154.9879 117.3629) (width 0.4) (layer F.Cu) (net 11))
 (segment (start 154.9879 117.3629) (end 155.675 118.05) (width 0.4) (layer F.Cu) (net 11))
 (segment (start 151.3351 106.6949) (end 151.335 106.695) (width 0.4) (layer F.Cu) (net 12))
 (segment (start 151.335 118.1195) (end 151.3351 118.1196) (width 0.4) (layer F.Cu) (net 12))
 (segment (start 151.3351 118.1196) (end 151.3351 120.4109) (width 0.4) (layer F.Cu) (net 12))
 (segment (start 151.335 118.1195) (end 151.335 106.695) (width 1) (layer F.Cu) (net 12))
 (segment (start 156.7 120.55) (end 151.474 120.55) (width 1) (layer F.Cu) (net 12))
 (segment (start 151.474 120.55) (end 151.335 120.411) (width 1) (layer F.Cu) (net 12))
 (segment (start 151.335 120.411) (end 151.335 118.1195) (width 1) (layer F.Cu) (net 12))
 (segment (start 154.0021 110.2509) (end 156.103 108.15) (width 1) (layer F.Cu) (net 13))
 (segment (start 156.103 108.15) (end 157.1 108.15) (width 1) (layer F.Cu) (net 13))
 (segment (start 154.002 110.251) (end 154.0021 110.2509) (width 1) (layer F.Cu) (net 13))
 (segment (start 157.1 108.15) (end 157.6 108.15) (width 1) (layer F.Cu) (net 13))
 (segment (start 157.6 108.15) (end 160.2 105.55) (width 1) (layer F.Cu) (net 13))
 (segment (start 164.75 105) (end 164.75 104.7) (width 1) (layer F.Cu) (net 1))
 (segment (start 164.75 104.7) (end 167.15 102.3) (width 1) (layer F.Cu) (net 1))
 (segment (start 182.61 123.19) (end 177.29 123.19) (width 1) (layer B.Cu) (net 1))
 (segment (start 177.29 123.19) (end 162.4 108.7) (width 1) (layer B.Cu) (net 1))
 (segment (start 162.4 108.7) (end 162.4 106.2) (width 1) (layer B.Cu) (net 1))
 (segment (start 162.4 106.2) (end 161.65 106.8) (width 1) (layer F.Cu) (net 1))
 (segment (start 161.65 106.8) (end 160.2 108.25) (width 1) (layer F.Cu) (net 1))
 (segment (start 162.4 106.2) (end 164.5 105) (width 1) (layer F.Cu) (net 1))
 (segment (start 164.5 105) (end 164.75 105) (width 1) (layer F.Cu) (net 1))
 (segment (start 182.61 123.19) (end 181.85 123.95) (width 1) (layer F.Cu) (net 1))
 (segment (start 181.85 123.95) (end 174.8 123.95) (width 1) (layer F.Cu) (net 1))
 (segment (start 166.025 116.5) (end 166.025 114.525) (width 0.4) (layer F.Cu) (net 1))
 (segment (start 166.025 114.525) (end 165.5 114) (width 0.4) (layer F.Cu) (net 1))
 (segment (start 165.5 114) (end 162.4 111.3) (width 0.4) (layer B.Cu) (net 1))
 (segment (start 162.4 111.3) (end 162.4 108.7) (width 0.4) (layer B.Cu) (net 1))
 (segment (start 157.25 111.8) (end 157.25 111.2) (width 1) (layer F.Cu) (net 1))
 (segment (start 157.25 111.2) (end 160.2 108.25) (width 1) (layer F.Cu) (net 1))
 (segment (start 162.4 106.2) (end 169.2 106.2) (width 0.4) (layer B.Cu) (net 1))
 (segment (start 169.2 106.2) (end 169.3 106.3) (width 0.4) (layer B.Cu) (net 1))
 (segment (start 169.3 106.3) (end 169.275 106.325) (width 0.4) (layer F.Cu) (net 1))
 (segment (start 169.275 106.325) (end 169.275 109.3) (width 0.4) (layer F.Cu) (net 1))
 (via (at 162.4 106.2) (size 0.6) (layers F.Cu B.Cu) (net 1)) (via (at 165.5 114) (size 0.6) (layers F.Cu B.Cu) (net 1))
 (via (at 169.3 106.3) (size 0.6) (layers F.Cu B.Cu) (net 1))
 (segment (start 164.075 116.5) (end 164.075 119.475) (width 0.4) (layer F.Cu) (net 14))
 (segment (start 164.075 119.475) (end 163.95 119.6) (width 0.4) (layer F.Cu) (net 14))
 (segment (start 174.8 121.25) (end 174.601 121.051) (width 1) (layer F.Cu) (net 2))
 (segment (start 174.601 121.051) (end 171.3 121.051) (width 1) (layer F.Cu) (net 2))
 (segment (start 178.88 100.33) (end 182.61 100.33) (width 1) (layer F.Cu) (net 3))
 (segment (start 182.61 100.33) (end 183.156 99.784) (width 1) (layer F.Cu) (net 3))
 (segment (start 183.156 99.784) (end 186.73 99.784) (width 1) (layer F.Cu) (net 3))
 (segment (start 178.88 102.87) (end 182.61 102.87) (width 1) (layer F.Cu) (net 4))
 (segment (start 182.61 102.87) (end 183.029 102.451) (width 1) (layer F.Cu) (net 4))
 (segment (start 183.029 102.451) (end 186.73 102.451) (width 1) (layer F.Cu) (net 4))
 (segment (start 178.88 105.41) (end 182.61 105.41) (width 1) (layer F.Cu) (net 5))
 (segment (start 182.61 105.41) (end 182.775 105.245) (width 1) (layer F.Cu) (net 5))
 (segment (start 182.775 105.245) (end 186.73 105.245) (width 1) (layer F.Cu) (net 5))
 (segment (start 178.88 107.95) (end 182.61 107.95) (width 1) (layer F.Cu) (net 6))
 (segment (start 182.61 107.95) (end 182.699 108.039) (width 1) (layer F.Cu) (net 6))
 (segment (start 182.699 108.039) (end 186.73 108.039) (width 1) (layer F.Cu) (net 6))
 (segment (start 178.88 110.49) (end 182.61 110.49) (width 1) (layer F.Cu) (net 7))
 (segment (start 182.61 110.49) (end 182.953 110.833) (width 1) (layer F.Cu) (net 7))
 (segment (start 182.953 110.833) (end 186.73 110.833) (width 1) (layer F.Cu) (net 7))
 (segment (start 178.88 113.03) (end 182.61 113.03) (width 1) (layer F.Cu) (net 8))
 (segment (start 182.61 113.03) (end 183.08 113.5) (width 1) (layer F.Cu) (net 8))
 (segment (start 183.08 113.5) (end 186.73 113.5) (width 1) (layer F.Cu) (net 8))
 (segment (start 178.88 115.57) (end 182.61 115.57) (width 1) (layer F.Cu) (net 9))
 (segment (start 182.61 115.57) (end 186.006 115.57) (width 1) (layer F.Cu) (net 9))
 (segment (start 186.006 115.57) (end 186.73 116.294) (width 1) (layer F.Cu) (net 9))
 (segment (start 178.88 118.11) (end 182.61 118.11) (width 1) (layer F.Cu) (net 10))
 (segment (start 182.61 118.11) (end 185.752 118.11) (width 1) (layer F.Cu) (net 10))
 (segment (start 185.752 118.11) (end 186.73 119.088) (width 1) (layer F.Cu) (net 10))
 (segment (start 154.0021 112.7911) (end 154.0021 112.7909) (width 0.4) (layer F.Cu) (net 25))
 (segment (start 154.0021 112.7911) (end 154.718 113.507) (width 0.4) (layer F.Cu) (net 25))
 (segment (start 154.718 113.507) (end 162.331 113.507) (width 0.4) (layer F.Cu) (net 25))
 (segment (start 162.331 113.507) (end 163.4 114.576) (width 0.4) (layer F.Cu) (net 25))
 (segment (start 163.4 114.576) (end 163.4 115.162) (width 0.4) (layer F.Cu) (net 25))
 (segment (start 163.4 115.162) (end 163.425 115.188) (width 0.4) (layer F.Cu) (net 25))
 (segment (start 163.425 115.188) (end 163.425 116.5) (width 0.4) (layer F.Cu) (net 25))
 (segment (start 154.002 112.791) (end 154.0021 112.7911) (width 0.4) (layer F.Cu) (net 25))
 (segment (start 154.002 114.823) (end 154.0021 114.8229) (width 0.4) (layer F.Cu) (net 24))
 (segment (start 154.0021 114.8229) (end 154.718 114.107) (width 0.4) (layer F.Cu) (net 24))
 (segment (start 154.718 114.107) (end 162.083 114.107) (width 0.4) (layer F.Cu) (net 24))
 (segment (start 162.083 114.107) (end 162.8 114.824) (width 0.4) (layer F.Cu) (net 24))
 (segment (start 162.8 114.824) (end 162.8 115.162) (width 0.4) (layer F.Cu) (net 24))
 (segment (start 162.8 115.162) (end 162.775 115.188) (width 0.4) (layer F.Cu) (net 24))
 (segment (start 162.775 115.188) (end 162.775 116.5) (width 0.4) (layer F.Cu) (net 24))
 (segment (start 159.95 111.8) (end 163.3 111.8) (width 0.4) (layer F.Cu) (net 15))
 (segment (start 163.3 111.8) (end 164.075 111.025) (width 0.4) (layer F.Cu) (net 15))
 (segment (start 164.075 111.025) (end 164.075 109.3) (width 0.4) (layer F.Cu) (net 15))
 (segment (start 172.2 100.3) (end 176.15 100.3) (width 0.4) (layer F.Cu) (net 16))
 (segment (start 176.15 100.3) (end 176.18 100.33) (width 0.4) (layer F.Cu) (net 16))
 (segment (start 171.225 109.3) (end 171.225 106.325) (width 0.4) (layer F.Cu) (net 16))
 (segment (start 171.225 106.325) (end 171.2 106.3) (width 0.4) (layer F.Cu) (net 16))
 (segment (start 171.2 106.3) (end 171.2 101.3) (width 0.4) (layer B.Cu) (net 16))
 (segment (start 171.2 101.3) (end 172.2 100.3) (width 0.4) (layer B.Cu) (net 16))
 (via (at 171.2 106.3) (size 0.6) (layers F.Cu B.Cu) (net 16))
 (via (at 172.2 100.3) (size 0.6) (layers F.Cu B.Cu) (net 16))
 (segment (start 176.18 102.87) (end 171.63 102.87) (width 0.4) (layer F.Cu) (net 19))
 (segment (start 171.63 102.87) (end 168.625 105.875) (width 0.4) (layer F.Cu) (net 19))
 (segment (start 168.625 105.875) (end 168.625 109.3) (width 0.4) (layer F.Cu) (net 19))
 (segment (start 169.925 109.3) (end 169.925 106.575) (width 0.4) (layer F.Cu) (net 18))
 (segment (start 169.925 106.575) (end 171.09 105.41) (width 0.4) (layer F.Cu) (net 18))
 (segment (start 171.09 105.41) (end 176.18 105.41) (width 0.4) (layer F.Cu) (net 18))
 (segment (start 165.6 107.5) (end 165.4 107.7) (width 0.4) (layer B.Cu) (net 23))
 (segment (start 165.6 107.5) (end 173.1 107.5) (width 0.4) (layer B.Cu) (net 23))
 (segment (start 164.725 109.3) (end 164.725 108.075) (width 0.4) (layer F.Cu) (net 23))
 (segment (start 164.725 108.075) (end 165.4 107.7) (width 0.4) (layer F.Cu) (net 23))
 (segment (start 173.1 107.5) (end 173.85 107.95) (width 0.4) (layer F.Cu) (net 23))
 (segment (start 173.85 107.95) (end 176.18 107.95) (width 0.4) (layer F.Cu) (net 23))
 (via (at 173.1 107.5) (size 0.6) (layers F.Cu B.Cu) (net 23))
 (via (at 165.4 107.7) (size 0.6) (layers F.Cu B.Cu) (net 23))
 (segment (start 170.575 109.3) (end 170.575 110.575) (width 0.4) (layer F.Cu) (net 17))
 (segment (start 170.575 110.575) (end 171 111) (width 0.4) (layer F.Cu) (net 17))
 (segment (start 171 111) (end 175.67 111) (width 0.4) (layer F.Cu) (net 17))
 (segment (start 175.67 111) (end 176.18 110.49) (width 0.4) (layer F.Cu) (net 17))
 (segment (start 176.18 113.03) (end 168.03 113.03) (width 0.4) (layer F.Cu) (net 21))
 (segment (start 168.03 113.03) (end 166.025 111.025) (width 0.4) (layer F.Cu) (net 21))
 (segment (start 166.025 111.025) (end 166.025 109.3) (width 0.4) (layer F.Cu) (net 21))
 (segment (start 176.18 115.57) (end 174.07 115.57) (width 0.4) (layer F.Cu) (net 22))
 (segment (start 174.07 115.57) (end 172.5 114) (width 0.4) (layer F.Cu) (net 22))
 (segment (start 172.5 114) (end 168 114) (width 0.4) (layer F.Cu) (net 22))
 (segment (start 168 114) (end 165.375 111.375) (width 0.4) (layer F.Cu) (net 22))
 (segment (start 165.375 111.375) (end 165.375 109.3) (width 0.4) (layer F.Cu) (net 22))
 (segment (start 174 116.7) (end 175.41 118.11) (width 0.4) (layer F.Cu) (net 20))
 (segment (start 175.41 118.11) (end 176.18 118.11) (width 0.4) (layer F.Cu) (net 20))
 (segment (start 167.975 109.3) (end 167.975 110.675) (width 0.4) (layer F.Cu) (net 20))
 (segment (start 167.975 110.675) (end 169 111.7) (width 0.4) (layer F.Cu) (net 20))
 (segment (start 169 111.7) (end 174 116.7) (width 0.4) (layer B.Cu) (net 20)) (via (at 174 116.7) (size 0.6) (layers F.Cu B.Cu) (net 20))
 (via (at 169 111.7) (size 0.6) (layers F.Cu B.Cu) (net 20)))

